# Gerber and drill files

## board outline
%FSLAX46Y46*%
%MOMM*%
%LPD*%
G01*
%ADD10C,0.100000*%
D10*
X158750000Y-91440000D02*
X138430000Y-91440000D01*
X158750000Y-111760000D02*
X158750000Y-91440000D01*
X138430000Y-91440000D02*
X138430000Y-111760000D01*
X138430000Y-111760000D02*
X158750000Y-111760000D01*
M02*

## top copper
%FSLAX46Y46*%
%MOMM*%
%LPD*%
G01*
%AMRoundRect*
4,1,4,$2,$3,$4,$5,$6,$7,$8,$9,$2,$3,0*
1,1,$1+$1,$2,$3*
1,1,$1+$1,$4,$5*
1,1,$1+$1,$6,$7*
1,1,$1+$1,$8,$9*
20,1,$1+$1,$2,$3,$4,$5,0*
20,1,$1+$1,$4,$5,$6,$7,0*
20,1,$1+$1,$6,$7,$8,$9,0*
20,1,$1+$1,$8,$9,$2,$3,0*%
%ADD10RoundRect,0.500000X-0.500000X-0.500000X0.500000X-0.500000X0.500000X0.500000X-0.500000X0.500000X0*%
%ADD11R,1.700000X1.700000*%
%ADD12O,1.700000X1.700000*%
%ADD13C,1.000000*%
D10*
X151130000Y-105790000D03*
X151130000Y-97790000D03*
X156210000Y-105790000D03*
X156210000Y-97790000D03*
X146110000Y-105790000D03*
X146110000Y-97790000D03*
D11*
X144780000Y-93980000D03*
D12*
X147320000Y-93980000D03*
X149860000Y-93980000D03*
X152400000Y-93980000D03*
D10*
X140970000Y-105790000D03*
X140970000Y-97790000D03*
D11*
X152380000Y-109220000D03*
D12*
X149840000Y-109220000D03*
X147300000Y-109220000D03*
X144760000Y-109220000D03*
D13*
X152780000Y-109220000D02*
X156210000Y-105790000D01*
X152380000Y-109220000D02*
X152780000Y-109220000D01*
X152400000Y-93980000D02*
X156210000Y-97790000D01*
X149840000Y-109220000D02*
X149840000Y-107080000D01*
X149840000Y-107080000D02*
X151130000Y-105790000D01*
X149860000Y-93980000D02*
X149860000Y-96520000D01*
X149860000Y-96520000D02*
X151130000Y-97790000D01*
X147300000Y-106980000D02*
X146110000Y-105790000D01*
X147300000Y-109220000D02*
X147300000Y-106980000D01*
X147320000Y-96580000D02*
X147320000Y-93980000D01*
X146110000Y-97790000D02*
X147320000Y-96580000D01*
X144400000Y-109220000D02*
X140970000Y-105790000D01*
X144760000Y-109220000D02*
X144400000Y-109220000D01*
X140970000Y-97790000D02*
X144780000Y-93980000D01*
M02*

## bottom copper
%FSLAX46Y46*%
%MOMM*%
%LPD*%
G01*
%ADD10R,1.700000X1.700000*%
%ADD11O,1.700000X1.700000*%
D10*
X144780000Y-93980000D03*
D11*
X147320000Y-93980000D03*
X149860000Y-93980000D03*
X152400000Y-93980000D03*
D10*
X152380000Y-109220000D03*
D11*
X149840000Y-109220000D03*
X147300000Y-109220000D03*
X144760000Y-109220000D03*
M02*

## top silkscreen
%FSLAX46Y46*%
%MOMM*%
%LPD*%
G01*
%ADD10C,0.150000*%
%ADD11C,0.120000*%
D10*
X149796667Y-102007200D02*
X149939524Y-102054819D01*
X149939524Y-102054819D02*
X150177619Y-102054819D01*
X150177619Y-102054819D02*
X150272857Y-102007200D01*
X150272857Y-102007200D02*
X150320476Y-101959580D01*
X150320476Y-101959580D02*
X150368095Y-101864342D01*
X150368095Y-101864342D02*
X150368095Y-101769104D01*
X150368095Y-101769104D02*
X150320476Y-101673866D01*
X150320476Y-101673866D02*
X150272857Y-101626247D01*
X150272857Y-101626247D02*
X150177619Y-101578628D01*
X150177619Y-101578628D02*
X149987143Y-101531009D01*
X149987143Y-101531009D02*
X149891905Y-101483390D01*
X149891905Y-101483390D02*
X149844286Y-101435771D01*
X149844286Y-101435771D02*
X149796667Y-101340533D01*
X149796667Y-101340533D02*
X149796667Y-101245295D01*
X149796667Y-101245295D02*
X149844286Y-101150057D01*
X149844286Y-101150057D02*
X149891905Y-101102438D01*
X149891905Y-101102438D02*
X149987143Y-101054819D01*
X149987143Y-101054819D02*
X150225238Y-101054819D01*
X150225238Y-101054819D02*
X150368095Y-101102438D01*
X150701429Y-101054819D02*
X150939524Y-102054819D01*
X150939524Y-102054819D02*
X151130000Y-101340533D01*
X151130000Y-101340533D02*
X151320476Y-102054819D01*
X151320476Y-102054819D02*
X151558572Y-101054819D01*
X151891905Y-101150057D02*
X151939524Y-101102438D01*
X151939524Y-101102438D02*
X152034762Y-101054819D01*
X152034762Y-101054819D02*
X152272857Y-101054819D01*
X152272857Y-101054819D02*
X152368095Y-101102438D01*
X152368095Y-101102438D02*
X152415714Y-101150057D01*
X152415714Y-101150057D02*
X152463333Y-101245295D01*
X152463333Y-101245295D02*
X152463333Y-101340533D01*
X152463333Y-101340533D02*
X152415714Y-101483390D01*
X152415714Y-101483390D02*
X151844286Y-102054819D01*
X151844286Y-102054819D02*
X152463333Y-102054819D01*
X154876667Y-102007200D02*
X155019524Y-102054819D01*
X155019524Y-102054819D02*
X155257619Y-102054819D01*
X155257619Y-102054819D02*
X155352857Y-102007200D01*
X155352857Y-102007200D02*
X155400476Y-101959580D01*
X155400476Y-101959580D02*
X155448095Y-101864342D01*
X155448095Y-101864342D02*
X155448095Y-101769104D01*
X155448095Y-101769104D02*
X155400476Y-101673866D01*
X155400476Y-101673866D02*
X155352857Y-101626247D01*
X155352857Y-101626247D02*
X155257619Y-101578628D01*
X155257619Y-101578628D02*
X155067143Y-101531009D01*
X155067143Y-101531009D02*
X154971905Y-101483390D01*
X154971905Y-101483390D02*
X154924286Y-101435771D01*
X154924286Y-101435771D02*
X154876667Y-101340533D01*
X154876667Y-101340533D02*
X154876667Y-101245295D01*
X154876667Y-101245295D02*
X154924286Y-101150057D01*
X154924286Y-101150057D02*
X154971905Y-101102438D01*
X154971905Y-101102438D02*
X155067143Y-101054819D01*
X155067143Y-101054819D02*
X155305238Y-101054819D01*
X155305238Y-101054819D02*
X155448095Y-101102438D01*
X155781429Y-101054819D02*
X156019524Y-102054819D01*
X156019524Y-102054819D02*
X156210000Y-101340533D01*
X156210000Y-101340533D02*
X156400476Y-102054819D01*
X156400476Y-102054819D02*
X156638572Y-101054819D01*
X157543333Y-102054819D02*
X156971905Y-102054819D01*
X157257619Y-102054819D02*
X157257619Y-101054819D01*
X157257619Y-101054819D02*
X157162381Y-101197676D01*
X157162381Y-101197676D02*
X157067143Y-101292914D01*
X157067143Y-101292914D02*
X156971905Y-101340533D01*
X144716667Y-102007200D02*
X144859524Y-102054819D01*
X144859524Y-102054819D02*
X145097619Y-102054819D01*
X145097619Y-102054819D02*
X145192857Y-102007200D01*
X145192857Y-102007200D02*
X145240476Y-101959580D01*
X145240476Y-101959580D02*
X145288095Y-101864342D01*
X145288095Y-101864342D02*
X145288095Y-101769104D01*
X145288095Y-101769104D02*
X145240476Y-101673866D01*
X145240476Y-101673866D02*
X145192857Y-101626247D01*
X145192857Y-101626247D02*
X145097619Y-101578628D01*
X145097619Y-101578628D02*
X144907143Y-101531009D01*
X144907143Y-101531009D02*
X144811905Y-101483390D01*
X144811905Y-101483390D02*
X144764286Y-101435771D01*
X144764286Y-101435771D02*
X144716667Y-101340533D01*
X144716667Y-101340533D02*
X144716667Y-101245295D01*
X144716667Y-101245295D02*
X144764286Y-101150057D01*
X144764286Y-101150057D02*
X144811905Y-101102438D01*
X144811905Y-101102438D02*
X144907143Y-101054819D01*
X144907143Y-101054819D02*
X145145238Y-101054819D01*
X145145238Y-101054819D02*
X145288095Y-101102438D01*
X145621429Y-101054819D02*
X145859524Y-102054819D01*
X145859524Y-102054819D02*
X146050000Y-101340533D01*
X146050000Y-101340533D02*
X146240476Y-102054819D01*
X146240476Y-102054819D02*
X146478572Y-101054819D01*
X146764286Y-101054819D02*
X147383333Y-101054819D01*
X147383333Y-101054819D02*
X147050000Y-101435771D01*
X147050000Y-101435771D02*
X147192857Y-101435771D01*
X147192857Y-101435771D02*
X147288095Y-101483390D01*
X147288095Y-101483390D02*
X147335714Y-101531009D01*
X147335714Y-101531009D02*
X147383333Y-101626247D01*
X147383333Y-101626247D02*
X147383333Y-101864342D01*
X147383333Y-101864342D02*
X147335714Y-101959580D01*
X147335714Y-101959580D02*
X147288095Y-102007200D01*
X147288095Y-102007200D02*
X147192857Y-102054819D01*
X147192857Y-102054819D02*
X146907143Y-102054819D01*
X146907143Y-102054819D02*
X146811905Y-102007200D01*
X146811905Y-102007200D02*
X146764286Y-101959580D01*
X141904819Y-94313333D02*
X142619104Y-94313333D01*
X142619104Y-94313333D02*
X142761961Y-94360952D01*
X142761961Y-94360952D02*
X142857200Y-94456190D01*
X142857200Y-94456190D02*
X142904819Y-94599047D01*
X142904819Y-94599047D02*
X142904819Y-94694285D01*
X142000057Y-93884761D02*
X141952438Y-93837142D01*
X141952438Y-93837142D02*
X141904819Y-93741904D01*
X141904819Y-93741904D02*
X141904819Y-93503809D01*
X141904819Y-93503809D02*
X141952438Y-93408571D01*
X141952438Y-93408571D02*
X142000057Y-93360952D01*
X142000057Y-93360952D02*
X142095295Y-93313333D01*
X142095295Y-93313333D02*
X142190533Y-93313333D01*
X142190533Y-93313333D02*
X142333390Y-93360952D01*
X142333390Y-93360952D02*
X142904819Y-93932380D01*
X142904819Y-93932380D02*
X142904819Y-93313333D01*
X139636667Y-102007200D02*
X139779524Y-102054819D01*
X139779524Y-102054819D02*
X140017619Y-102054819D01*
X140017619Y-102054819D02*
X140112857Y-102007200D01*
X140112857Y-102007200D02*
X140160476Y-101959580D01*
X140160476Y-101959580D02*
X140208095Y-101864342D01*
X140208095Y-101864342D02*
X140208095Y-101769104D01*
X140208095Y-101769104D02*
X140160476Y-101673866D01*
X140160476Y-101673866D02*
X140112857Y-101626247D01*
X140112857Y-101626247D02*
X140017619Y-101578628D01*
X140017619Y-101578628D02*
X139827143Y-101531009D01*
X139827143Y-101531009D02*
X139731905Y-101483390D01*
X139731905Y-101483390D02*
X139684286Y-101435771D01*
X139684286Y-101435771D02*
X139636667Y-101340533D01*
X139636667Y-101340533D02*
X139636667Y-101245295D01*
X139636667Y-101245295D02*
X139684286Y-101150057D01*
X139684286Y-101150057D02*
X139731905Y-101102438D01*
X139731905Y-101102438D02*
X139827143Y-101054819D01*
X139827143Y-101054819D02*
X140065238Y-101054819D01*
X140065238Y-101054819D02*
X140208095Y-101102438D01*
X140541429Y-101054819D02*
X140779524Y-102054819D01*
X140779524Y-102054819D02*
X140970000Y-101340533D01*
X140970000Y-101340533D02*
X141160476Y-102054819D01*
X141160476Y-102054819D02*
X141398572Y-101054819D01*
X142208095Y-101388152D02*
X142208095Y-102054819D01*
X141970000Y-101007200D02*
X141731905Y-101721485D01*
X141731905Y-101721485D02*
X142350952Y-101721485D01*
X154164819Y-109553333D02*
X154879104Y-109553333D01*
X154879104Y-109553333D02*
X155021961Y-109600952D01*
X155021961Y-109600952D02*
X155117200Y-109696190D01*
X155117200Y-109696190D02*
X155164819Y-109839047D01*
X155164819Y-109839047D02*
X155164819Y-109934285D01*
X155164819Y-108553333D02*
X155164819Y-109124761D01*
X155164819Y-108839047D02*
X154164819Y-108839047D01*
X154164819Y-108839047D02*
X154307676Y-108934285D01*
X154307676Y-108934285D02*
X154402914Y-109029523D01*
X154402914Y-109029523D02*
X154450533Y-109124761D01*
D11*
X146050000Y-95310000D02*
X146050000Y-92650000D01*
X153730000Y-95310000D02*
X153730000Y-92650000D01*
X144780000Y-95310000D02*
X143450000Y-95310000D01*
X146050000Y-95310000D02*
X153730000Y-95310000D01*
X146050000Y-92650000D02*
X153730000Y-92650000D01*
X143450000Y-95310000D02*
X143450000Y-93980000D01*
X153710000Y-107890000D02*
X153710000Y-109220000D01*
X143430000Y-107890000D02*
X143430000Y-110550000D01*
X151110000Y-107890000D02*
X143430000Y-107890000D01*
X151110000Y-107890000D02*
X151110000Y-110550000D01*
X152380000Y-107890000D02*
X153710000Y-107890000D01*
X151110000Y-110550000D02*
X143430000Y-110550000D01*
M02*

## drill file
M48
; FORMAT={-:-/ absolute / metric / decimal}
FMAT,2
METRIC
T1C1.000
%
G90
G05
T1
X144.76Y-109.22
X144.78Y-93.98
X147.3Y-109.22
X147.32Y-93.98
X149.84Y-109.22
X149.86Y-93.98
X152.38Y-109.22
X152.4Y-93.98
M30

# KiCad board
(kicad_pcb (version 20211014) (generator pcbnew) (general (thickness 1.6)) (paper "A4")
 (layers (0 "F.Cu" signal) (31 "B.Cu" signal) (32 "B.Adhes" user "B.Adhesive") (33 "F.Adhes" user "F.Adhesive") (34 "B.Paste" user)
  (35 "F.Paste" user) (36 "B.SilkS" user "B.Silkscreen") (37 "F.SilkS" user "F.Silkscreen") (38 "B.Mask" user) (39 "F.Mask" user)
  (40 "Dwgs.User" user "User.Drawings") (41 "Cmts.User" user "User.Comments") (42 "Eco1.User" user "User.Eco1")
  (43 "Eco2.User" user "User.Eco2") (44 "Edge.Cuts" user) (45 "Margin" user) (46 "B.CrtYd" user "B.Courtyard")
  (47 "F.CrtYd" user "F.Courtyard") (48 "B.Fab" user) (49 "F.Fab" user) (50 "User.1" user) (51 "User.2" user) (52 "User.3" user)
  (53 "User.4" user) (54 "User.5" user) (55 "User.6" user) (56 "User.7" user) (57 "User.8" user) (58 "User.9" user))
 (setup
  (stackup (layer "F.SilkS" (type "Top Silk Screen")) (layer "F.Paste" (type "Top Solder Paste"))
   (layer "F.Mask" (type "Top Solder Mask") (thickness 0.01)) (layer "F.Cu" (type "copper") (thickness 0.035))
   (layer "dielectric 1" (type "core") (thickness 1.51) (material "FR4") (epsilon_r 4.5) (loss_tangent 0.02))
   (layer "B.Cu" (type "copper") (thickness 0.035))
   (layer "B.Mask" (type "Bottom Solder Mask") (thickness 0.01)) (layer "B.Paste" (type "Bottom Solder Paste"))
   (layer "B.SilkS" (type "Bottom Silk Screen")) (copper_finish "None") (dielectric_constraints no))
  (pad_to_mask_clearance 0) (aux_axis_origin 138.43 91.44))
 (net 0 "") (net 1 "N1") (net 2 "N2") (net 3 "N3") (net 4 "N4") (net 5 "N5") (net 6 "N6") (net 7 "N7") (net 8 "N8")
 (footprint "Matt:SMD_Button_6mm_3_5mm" (layer "F.Cu") (at 151.13 105.79)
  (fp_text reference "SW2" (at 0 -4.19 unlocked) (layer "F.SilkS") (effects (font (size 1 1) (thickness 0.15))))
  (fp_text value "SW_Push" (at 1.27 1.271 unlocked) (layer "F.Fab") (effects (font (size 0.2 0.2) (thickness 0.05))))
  (pad "1" smd roundrect (at 0 0) (size 2 2) (layers "F.Cu" "F.Paste" "F.Mask") (roundrect_rratio 0.25) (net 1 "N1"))
  (pad "2" smd roundrect (at 0 -8) (size 2 2) (layers "F.Cu" "F.Paste" "F.Mask") (roundrect_rratio 0.25) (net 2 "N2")))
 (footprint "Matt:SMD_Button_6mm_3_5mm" (layer "F.Cu") (at 156.21 105.79)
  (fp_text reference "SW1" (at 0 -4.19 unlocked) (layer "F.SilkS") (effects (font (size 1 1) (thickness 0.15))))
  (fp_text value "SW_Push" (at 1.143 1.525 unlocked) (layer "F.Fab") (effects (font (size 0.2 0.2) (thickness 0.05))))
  (pad "1" smd roundrect (at 0 0) (size 2 2) (layers "F.Cu" "F.Paste" "F.Mask") (roundrect_rratio 0.25) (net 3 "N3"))
  (pad "2" smd roundrect (at 0 -8) (size 2 2) (layers "F.Cu" "F.Paste" "F.Mask") (roundrect_rratio 0.25) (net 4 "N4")))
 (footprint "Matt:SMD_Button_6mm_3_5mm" (layer "F.Cu") (at 146.11 105.79)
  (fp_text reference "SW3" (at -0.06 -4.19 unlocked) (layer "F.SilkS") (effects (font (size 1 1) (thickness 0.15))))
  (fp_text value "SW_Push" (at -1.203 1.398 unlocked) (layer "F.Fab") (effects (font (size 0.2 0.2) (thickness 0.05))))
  (pad "1" smd roundrect (at 0 0) (size 2 2) (layers "F.Cu" "F.Paste" "F.Mask") (roundrect_rratio 0.25) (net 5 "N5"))
  (pad "2" smd roundrect (at 0 -8) (size 2 2) (layers "F.Cu" "F.Paste" "F.Mask") (roundrect_rratio 0.25) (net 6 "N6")))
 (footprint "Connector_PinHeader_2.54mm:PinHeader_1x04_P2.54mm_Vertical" (layer "F.Cu") (at 144.78 93.98 90)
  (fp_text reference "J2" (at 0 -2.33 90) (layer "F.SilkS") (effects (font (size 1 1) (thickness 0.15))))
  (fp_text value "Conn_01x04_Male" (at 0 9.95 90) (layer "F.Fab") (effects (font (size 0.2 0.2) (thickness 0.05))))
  (fp_line (start -1.33 1.27) (end 1.33 1.27) (layer "F.SilkS") (width 0.12))
  (fp_line (start -1.33 8.95) (end 1.33 8.95) (layer "F.SilkS") (width 0.12))
  (fp_line (start -1.33 0) (end -1.33 -1.33) (layer "F.SilkS") (width 0.12))
  (fp_line (start -1.33 1.27) (end -1.33 8.95) (layer "F.SilkS") (width 0.12))
  (fp_line (start 1.33 1.27) (end 1.33 8.95) (layer "F.SilkS") (width 0.12))
  (fp_line (start -1.33 -1.33) (end 0 -1.33) (layer "F.SilkS") (width 0.12))
  (pad "1" thru_hole rect (at 0 0 90) (size 1.7 1.7) (drill 1) (layers *.Cu *.Mask) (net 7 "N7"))
  (pad "2" thru_hole oval (at 0 2.54 90) (size 1.7 1.7) (drill 1) (layers *.Cu *.Mask) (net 6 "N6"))
  (pad "3" thru_hole oval (at 0 5.08 90) (size 1.7 1.7) (drill 1) (layers *.Cu *.Mask) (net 2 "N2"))
  (pad "4" thru_hole oval (at 0 7.62 90) (size 1.7 1.7) (drill 1) (layers *.Cu *.Mask) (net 4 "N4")))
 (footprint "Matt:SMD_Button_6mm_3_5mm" (layer "F.Cu") (at 140.97 105.79)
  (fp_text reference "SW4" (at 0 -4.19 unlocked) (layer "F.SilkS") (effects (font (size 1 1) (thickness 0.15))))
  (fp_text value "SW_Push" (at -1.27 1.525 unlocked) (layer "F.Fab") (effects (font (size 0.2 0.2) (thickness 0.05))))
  (pad "1" smd roundrect (at 0 0) (size 2 2) (layers "F.Cu" "F.Paste" "F.Mask") (roundrect_rratio 0.25) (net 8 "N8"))
  (pad "2" smd roundrect (at 0 -8) (size 2 2) (layers "F.Cu" "F.Paste" "F.Mask") (roundrect_rratio 0.25) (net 7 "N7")))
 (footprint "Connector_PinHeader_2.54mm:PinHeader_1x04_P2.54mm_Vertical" (layer "F.Cu") (at 152.38 109.22 -90)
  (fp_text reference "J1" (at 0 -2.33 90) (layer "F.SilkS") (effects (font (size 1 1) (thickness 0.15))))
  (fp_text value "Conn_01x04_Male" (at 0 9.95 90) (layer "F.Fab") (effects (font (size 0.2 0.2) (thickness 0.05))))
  (fp_line (start -1.33 -1.33) (end 0 -1.33) (layer "F.SilkS") (width 0.12))
  (fp_line (start -1.33 8.95) (end 1.33 8.95) (layer "F.SilkS") (width 0.12))
  (fp_line (start -1.33 1.27) (end -1.33 8.95) (layer "F.SilkS") (width 0.12))
  (fp_line (start -1.33 1.27) (end 1.33 1.27) (layer "F.SilkS") (width 0.12))
  (fp_line (start -1.33 0) (end -1.33 -1.33) (layer "F.SilkS") (width 0.12))
  (fp_line (start 1.33 1.27) (end 1.33 8.95) (layer "F.SilkS") (width 0.12))
  (pad "1" thru_hole rect (at 0 0 270) (size 1.7 1.7) (drill 1) (layers *.Cu *.Mask) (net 3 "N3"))
  (pad "2" thru_hole oval (at 0 2.54 270) (size 1.7 1.7) (drill 1) (layers *.Cu *.Mask) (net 1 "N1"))
  (pad "3" thru_hole oval (at 0 5.08 270) (size 1.7 1.7) (drill 1) (layers *.Cu *.Mask) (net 5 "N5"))
  (pad "4" thru_hole oval (at 0 7.62 270) (size 1.7 1.7) (drill 1) (layers *.Cu *.Mask) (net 8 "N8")))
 (gr_line (start 158.75 91.44) (end 138.43 91.44) (layer "Edge.Cuts") (width 0.1))
 (gr_line (start 158.75 111.76) (end 158.75 91.44) (layer "Edge.Cuts") (width 0.1))
 (gr_line (start 138.43 91.44) (end 138.43 111.76) (layer "Edge.Cuts") (width 0.1))
 (gr_line (start 138.43 111.76) (end 158.75 111.76) (layer "Edge.Cuts") (width 0.1))
 (segment (start 152.78 109.22) (end 156.21 105.79) (width 1) (layer "F.Cu") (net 3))
 (segment (start 152.38 109.22) (end 152.78 109.22) (width 1) (layer "F.Cu") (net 3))
 (segment (start 152.4 93.98) (end 156.21 97.79) (width 1) (layer "F.Cu") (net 4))
 (segment (start 149.84 109.22) (end 149.84 107.08) (width 1) (layer "F.Cu") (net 1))
 (segment (start 149.84 107.08) (end 151.13 105.79) (width 1) (layer "F.Cu") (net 1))
 (segment (start 149.86 93.98) (end 149.86 96.52) (width 1) (layer "F.Cu") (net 2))
 (segment (start 149.86 96.52) (end 151.13 97.79) (width 1) (layer "F.Cu") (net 2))
 (segment (start 147.3 106.98) (end 146.11 105.79) (width 1) (layer "F.Cu") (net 5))
 (segment (start 147.3 109.22) (end 147.3 106.98) (width 1) (layer "F.Cu") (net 5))
 (segment (start 147.32 96.58) (end 147.32 93.98) (width 1) (layer "F.Cu") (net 6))
 (segment (start 146.11 97.79) (end 147.32 96.58) (width 1) (layer "F.Cu") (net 6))
 (segment (start 144.4 109.22) (end 140.97 105.79) (width 1) (layer "F.Cu") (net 8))
 (segment (start 144.76 109.22) (end 144.4 109.22) (width 1) (layer "F.Cu") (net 8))
 (segment (start 140.97 97.79) (end 144.78 93.98) (width 1) (layer "F.Cu") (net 7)))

